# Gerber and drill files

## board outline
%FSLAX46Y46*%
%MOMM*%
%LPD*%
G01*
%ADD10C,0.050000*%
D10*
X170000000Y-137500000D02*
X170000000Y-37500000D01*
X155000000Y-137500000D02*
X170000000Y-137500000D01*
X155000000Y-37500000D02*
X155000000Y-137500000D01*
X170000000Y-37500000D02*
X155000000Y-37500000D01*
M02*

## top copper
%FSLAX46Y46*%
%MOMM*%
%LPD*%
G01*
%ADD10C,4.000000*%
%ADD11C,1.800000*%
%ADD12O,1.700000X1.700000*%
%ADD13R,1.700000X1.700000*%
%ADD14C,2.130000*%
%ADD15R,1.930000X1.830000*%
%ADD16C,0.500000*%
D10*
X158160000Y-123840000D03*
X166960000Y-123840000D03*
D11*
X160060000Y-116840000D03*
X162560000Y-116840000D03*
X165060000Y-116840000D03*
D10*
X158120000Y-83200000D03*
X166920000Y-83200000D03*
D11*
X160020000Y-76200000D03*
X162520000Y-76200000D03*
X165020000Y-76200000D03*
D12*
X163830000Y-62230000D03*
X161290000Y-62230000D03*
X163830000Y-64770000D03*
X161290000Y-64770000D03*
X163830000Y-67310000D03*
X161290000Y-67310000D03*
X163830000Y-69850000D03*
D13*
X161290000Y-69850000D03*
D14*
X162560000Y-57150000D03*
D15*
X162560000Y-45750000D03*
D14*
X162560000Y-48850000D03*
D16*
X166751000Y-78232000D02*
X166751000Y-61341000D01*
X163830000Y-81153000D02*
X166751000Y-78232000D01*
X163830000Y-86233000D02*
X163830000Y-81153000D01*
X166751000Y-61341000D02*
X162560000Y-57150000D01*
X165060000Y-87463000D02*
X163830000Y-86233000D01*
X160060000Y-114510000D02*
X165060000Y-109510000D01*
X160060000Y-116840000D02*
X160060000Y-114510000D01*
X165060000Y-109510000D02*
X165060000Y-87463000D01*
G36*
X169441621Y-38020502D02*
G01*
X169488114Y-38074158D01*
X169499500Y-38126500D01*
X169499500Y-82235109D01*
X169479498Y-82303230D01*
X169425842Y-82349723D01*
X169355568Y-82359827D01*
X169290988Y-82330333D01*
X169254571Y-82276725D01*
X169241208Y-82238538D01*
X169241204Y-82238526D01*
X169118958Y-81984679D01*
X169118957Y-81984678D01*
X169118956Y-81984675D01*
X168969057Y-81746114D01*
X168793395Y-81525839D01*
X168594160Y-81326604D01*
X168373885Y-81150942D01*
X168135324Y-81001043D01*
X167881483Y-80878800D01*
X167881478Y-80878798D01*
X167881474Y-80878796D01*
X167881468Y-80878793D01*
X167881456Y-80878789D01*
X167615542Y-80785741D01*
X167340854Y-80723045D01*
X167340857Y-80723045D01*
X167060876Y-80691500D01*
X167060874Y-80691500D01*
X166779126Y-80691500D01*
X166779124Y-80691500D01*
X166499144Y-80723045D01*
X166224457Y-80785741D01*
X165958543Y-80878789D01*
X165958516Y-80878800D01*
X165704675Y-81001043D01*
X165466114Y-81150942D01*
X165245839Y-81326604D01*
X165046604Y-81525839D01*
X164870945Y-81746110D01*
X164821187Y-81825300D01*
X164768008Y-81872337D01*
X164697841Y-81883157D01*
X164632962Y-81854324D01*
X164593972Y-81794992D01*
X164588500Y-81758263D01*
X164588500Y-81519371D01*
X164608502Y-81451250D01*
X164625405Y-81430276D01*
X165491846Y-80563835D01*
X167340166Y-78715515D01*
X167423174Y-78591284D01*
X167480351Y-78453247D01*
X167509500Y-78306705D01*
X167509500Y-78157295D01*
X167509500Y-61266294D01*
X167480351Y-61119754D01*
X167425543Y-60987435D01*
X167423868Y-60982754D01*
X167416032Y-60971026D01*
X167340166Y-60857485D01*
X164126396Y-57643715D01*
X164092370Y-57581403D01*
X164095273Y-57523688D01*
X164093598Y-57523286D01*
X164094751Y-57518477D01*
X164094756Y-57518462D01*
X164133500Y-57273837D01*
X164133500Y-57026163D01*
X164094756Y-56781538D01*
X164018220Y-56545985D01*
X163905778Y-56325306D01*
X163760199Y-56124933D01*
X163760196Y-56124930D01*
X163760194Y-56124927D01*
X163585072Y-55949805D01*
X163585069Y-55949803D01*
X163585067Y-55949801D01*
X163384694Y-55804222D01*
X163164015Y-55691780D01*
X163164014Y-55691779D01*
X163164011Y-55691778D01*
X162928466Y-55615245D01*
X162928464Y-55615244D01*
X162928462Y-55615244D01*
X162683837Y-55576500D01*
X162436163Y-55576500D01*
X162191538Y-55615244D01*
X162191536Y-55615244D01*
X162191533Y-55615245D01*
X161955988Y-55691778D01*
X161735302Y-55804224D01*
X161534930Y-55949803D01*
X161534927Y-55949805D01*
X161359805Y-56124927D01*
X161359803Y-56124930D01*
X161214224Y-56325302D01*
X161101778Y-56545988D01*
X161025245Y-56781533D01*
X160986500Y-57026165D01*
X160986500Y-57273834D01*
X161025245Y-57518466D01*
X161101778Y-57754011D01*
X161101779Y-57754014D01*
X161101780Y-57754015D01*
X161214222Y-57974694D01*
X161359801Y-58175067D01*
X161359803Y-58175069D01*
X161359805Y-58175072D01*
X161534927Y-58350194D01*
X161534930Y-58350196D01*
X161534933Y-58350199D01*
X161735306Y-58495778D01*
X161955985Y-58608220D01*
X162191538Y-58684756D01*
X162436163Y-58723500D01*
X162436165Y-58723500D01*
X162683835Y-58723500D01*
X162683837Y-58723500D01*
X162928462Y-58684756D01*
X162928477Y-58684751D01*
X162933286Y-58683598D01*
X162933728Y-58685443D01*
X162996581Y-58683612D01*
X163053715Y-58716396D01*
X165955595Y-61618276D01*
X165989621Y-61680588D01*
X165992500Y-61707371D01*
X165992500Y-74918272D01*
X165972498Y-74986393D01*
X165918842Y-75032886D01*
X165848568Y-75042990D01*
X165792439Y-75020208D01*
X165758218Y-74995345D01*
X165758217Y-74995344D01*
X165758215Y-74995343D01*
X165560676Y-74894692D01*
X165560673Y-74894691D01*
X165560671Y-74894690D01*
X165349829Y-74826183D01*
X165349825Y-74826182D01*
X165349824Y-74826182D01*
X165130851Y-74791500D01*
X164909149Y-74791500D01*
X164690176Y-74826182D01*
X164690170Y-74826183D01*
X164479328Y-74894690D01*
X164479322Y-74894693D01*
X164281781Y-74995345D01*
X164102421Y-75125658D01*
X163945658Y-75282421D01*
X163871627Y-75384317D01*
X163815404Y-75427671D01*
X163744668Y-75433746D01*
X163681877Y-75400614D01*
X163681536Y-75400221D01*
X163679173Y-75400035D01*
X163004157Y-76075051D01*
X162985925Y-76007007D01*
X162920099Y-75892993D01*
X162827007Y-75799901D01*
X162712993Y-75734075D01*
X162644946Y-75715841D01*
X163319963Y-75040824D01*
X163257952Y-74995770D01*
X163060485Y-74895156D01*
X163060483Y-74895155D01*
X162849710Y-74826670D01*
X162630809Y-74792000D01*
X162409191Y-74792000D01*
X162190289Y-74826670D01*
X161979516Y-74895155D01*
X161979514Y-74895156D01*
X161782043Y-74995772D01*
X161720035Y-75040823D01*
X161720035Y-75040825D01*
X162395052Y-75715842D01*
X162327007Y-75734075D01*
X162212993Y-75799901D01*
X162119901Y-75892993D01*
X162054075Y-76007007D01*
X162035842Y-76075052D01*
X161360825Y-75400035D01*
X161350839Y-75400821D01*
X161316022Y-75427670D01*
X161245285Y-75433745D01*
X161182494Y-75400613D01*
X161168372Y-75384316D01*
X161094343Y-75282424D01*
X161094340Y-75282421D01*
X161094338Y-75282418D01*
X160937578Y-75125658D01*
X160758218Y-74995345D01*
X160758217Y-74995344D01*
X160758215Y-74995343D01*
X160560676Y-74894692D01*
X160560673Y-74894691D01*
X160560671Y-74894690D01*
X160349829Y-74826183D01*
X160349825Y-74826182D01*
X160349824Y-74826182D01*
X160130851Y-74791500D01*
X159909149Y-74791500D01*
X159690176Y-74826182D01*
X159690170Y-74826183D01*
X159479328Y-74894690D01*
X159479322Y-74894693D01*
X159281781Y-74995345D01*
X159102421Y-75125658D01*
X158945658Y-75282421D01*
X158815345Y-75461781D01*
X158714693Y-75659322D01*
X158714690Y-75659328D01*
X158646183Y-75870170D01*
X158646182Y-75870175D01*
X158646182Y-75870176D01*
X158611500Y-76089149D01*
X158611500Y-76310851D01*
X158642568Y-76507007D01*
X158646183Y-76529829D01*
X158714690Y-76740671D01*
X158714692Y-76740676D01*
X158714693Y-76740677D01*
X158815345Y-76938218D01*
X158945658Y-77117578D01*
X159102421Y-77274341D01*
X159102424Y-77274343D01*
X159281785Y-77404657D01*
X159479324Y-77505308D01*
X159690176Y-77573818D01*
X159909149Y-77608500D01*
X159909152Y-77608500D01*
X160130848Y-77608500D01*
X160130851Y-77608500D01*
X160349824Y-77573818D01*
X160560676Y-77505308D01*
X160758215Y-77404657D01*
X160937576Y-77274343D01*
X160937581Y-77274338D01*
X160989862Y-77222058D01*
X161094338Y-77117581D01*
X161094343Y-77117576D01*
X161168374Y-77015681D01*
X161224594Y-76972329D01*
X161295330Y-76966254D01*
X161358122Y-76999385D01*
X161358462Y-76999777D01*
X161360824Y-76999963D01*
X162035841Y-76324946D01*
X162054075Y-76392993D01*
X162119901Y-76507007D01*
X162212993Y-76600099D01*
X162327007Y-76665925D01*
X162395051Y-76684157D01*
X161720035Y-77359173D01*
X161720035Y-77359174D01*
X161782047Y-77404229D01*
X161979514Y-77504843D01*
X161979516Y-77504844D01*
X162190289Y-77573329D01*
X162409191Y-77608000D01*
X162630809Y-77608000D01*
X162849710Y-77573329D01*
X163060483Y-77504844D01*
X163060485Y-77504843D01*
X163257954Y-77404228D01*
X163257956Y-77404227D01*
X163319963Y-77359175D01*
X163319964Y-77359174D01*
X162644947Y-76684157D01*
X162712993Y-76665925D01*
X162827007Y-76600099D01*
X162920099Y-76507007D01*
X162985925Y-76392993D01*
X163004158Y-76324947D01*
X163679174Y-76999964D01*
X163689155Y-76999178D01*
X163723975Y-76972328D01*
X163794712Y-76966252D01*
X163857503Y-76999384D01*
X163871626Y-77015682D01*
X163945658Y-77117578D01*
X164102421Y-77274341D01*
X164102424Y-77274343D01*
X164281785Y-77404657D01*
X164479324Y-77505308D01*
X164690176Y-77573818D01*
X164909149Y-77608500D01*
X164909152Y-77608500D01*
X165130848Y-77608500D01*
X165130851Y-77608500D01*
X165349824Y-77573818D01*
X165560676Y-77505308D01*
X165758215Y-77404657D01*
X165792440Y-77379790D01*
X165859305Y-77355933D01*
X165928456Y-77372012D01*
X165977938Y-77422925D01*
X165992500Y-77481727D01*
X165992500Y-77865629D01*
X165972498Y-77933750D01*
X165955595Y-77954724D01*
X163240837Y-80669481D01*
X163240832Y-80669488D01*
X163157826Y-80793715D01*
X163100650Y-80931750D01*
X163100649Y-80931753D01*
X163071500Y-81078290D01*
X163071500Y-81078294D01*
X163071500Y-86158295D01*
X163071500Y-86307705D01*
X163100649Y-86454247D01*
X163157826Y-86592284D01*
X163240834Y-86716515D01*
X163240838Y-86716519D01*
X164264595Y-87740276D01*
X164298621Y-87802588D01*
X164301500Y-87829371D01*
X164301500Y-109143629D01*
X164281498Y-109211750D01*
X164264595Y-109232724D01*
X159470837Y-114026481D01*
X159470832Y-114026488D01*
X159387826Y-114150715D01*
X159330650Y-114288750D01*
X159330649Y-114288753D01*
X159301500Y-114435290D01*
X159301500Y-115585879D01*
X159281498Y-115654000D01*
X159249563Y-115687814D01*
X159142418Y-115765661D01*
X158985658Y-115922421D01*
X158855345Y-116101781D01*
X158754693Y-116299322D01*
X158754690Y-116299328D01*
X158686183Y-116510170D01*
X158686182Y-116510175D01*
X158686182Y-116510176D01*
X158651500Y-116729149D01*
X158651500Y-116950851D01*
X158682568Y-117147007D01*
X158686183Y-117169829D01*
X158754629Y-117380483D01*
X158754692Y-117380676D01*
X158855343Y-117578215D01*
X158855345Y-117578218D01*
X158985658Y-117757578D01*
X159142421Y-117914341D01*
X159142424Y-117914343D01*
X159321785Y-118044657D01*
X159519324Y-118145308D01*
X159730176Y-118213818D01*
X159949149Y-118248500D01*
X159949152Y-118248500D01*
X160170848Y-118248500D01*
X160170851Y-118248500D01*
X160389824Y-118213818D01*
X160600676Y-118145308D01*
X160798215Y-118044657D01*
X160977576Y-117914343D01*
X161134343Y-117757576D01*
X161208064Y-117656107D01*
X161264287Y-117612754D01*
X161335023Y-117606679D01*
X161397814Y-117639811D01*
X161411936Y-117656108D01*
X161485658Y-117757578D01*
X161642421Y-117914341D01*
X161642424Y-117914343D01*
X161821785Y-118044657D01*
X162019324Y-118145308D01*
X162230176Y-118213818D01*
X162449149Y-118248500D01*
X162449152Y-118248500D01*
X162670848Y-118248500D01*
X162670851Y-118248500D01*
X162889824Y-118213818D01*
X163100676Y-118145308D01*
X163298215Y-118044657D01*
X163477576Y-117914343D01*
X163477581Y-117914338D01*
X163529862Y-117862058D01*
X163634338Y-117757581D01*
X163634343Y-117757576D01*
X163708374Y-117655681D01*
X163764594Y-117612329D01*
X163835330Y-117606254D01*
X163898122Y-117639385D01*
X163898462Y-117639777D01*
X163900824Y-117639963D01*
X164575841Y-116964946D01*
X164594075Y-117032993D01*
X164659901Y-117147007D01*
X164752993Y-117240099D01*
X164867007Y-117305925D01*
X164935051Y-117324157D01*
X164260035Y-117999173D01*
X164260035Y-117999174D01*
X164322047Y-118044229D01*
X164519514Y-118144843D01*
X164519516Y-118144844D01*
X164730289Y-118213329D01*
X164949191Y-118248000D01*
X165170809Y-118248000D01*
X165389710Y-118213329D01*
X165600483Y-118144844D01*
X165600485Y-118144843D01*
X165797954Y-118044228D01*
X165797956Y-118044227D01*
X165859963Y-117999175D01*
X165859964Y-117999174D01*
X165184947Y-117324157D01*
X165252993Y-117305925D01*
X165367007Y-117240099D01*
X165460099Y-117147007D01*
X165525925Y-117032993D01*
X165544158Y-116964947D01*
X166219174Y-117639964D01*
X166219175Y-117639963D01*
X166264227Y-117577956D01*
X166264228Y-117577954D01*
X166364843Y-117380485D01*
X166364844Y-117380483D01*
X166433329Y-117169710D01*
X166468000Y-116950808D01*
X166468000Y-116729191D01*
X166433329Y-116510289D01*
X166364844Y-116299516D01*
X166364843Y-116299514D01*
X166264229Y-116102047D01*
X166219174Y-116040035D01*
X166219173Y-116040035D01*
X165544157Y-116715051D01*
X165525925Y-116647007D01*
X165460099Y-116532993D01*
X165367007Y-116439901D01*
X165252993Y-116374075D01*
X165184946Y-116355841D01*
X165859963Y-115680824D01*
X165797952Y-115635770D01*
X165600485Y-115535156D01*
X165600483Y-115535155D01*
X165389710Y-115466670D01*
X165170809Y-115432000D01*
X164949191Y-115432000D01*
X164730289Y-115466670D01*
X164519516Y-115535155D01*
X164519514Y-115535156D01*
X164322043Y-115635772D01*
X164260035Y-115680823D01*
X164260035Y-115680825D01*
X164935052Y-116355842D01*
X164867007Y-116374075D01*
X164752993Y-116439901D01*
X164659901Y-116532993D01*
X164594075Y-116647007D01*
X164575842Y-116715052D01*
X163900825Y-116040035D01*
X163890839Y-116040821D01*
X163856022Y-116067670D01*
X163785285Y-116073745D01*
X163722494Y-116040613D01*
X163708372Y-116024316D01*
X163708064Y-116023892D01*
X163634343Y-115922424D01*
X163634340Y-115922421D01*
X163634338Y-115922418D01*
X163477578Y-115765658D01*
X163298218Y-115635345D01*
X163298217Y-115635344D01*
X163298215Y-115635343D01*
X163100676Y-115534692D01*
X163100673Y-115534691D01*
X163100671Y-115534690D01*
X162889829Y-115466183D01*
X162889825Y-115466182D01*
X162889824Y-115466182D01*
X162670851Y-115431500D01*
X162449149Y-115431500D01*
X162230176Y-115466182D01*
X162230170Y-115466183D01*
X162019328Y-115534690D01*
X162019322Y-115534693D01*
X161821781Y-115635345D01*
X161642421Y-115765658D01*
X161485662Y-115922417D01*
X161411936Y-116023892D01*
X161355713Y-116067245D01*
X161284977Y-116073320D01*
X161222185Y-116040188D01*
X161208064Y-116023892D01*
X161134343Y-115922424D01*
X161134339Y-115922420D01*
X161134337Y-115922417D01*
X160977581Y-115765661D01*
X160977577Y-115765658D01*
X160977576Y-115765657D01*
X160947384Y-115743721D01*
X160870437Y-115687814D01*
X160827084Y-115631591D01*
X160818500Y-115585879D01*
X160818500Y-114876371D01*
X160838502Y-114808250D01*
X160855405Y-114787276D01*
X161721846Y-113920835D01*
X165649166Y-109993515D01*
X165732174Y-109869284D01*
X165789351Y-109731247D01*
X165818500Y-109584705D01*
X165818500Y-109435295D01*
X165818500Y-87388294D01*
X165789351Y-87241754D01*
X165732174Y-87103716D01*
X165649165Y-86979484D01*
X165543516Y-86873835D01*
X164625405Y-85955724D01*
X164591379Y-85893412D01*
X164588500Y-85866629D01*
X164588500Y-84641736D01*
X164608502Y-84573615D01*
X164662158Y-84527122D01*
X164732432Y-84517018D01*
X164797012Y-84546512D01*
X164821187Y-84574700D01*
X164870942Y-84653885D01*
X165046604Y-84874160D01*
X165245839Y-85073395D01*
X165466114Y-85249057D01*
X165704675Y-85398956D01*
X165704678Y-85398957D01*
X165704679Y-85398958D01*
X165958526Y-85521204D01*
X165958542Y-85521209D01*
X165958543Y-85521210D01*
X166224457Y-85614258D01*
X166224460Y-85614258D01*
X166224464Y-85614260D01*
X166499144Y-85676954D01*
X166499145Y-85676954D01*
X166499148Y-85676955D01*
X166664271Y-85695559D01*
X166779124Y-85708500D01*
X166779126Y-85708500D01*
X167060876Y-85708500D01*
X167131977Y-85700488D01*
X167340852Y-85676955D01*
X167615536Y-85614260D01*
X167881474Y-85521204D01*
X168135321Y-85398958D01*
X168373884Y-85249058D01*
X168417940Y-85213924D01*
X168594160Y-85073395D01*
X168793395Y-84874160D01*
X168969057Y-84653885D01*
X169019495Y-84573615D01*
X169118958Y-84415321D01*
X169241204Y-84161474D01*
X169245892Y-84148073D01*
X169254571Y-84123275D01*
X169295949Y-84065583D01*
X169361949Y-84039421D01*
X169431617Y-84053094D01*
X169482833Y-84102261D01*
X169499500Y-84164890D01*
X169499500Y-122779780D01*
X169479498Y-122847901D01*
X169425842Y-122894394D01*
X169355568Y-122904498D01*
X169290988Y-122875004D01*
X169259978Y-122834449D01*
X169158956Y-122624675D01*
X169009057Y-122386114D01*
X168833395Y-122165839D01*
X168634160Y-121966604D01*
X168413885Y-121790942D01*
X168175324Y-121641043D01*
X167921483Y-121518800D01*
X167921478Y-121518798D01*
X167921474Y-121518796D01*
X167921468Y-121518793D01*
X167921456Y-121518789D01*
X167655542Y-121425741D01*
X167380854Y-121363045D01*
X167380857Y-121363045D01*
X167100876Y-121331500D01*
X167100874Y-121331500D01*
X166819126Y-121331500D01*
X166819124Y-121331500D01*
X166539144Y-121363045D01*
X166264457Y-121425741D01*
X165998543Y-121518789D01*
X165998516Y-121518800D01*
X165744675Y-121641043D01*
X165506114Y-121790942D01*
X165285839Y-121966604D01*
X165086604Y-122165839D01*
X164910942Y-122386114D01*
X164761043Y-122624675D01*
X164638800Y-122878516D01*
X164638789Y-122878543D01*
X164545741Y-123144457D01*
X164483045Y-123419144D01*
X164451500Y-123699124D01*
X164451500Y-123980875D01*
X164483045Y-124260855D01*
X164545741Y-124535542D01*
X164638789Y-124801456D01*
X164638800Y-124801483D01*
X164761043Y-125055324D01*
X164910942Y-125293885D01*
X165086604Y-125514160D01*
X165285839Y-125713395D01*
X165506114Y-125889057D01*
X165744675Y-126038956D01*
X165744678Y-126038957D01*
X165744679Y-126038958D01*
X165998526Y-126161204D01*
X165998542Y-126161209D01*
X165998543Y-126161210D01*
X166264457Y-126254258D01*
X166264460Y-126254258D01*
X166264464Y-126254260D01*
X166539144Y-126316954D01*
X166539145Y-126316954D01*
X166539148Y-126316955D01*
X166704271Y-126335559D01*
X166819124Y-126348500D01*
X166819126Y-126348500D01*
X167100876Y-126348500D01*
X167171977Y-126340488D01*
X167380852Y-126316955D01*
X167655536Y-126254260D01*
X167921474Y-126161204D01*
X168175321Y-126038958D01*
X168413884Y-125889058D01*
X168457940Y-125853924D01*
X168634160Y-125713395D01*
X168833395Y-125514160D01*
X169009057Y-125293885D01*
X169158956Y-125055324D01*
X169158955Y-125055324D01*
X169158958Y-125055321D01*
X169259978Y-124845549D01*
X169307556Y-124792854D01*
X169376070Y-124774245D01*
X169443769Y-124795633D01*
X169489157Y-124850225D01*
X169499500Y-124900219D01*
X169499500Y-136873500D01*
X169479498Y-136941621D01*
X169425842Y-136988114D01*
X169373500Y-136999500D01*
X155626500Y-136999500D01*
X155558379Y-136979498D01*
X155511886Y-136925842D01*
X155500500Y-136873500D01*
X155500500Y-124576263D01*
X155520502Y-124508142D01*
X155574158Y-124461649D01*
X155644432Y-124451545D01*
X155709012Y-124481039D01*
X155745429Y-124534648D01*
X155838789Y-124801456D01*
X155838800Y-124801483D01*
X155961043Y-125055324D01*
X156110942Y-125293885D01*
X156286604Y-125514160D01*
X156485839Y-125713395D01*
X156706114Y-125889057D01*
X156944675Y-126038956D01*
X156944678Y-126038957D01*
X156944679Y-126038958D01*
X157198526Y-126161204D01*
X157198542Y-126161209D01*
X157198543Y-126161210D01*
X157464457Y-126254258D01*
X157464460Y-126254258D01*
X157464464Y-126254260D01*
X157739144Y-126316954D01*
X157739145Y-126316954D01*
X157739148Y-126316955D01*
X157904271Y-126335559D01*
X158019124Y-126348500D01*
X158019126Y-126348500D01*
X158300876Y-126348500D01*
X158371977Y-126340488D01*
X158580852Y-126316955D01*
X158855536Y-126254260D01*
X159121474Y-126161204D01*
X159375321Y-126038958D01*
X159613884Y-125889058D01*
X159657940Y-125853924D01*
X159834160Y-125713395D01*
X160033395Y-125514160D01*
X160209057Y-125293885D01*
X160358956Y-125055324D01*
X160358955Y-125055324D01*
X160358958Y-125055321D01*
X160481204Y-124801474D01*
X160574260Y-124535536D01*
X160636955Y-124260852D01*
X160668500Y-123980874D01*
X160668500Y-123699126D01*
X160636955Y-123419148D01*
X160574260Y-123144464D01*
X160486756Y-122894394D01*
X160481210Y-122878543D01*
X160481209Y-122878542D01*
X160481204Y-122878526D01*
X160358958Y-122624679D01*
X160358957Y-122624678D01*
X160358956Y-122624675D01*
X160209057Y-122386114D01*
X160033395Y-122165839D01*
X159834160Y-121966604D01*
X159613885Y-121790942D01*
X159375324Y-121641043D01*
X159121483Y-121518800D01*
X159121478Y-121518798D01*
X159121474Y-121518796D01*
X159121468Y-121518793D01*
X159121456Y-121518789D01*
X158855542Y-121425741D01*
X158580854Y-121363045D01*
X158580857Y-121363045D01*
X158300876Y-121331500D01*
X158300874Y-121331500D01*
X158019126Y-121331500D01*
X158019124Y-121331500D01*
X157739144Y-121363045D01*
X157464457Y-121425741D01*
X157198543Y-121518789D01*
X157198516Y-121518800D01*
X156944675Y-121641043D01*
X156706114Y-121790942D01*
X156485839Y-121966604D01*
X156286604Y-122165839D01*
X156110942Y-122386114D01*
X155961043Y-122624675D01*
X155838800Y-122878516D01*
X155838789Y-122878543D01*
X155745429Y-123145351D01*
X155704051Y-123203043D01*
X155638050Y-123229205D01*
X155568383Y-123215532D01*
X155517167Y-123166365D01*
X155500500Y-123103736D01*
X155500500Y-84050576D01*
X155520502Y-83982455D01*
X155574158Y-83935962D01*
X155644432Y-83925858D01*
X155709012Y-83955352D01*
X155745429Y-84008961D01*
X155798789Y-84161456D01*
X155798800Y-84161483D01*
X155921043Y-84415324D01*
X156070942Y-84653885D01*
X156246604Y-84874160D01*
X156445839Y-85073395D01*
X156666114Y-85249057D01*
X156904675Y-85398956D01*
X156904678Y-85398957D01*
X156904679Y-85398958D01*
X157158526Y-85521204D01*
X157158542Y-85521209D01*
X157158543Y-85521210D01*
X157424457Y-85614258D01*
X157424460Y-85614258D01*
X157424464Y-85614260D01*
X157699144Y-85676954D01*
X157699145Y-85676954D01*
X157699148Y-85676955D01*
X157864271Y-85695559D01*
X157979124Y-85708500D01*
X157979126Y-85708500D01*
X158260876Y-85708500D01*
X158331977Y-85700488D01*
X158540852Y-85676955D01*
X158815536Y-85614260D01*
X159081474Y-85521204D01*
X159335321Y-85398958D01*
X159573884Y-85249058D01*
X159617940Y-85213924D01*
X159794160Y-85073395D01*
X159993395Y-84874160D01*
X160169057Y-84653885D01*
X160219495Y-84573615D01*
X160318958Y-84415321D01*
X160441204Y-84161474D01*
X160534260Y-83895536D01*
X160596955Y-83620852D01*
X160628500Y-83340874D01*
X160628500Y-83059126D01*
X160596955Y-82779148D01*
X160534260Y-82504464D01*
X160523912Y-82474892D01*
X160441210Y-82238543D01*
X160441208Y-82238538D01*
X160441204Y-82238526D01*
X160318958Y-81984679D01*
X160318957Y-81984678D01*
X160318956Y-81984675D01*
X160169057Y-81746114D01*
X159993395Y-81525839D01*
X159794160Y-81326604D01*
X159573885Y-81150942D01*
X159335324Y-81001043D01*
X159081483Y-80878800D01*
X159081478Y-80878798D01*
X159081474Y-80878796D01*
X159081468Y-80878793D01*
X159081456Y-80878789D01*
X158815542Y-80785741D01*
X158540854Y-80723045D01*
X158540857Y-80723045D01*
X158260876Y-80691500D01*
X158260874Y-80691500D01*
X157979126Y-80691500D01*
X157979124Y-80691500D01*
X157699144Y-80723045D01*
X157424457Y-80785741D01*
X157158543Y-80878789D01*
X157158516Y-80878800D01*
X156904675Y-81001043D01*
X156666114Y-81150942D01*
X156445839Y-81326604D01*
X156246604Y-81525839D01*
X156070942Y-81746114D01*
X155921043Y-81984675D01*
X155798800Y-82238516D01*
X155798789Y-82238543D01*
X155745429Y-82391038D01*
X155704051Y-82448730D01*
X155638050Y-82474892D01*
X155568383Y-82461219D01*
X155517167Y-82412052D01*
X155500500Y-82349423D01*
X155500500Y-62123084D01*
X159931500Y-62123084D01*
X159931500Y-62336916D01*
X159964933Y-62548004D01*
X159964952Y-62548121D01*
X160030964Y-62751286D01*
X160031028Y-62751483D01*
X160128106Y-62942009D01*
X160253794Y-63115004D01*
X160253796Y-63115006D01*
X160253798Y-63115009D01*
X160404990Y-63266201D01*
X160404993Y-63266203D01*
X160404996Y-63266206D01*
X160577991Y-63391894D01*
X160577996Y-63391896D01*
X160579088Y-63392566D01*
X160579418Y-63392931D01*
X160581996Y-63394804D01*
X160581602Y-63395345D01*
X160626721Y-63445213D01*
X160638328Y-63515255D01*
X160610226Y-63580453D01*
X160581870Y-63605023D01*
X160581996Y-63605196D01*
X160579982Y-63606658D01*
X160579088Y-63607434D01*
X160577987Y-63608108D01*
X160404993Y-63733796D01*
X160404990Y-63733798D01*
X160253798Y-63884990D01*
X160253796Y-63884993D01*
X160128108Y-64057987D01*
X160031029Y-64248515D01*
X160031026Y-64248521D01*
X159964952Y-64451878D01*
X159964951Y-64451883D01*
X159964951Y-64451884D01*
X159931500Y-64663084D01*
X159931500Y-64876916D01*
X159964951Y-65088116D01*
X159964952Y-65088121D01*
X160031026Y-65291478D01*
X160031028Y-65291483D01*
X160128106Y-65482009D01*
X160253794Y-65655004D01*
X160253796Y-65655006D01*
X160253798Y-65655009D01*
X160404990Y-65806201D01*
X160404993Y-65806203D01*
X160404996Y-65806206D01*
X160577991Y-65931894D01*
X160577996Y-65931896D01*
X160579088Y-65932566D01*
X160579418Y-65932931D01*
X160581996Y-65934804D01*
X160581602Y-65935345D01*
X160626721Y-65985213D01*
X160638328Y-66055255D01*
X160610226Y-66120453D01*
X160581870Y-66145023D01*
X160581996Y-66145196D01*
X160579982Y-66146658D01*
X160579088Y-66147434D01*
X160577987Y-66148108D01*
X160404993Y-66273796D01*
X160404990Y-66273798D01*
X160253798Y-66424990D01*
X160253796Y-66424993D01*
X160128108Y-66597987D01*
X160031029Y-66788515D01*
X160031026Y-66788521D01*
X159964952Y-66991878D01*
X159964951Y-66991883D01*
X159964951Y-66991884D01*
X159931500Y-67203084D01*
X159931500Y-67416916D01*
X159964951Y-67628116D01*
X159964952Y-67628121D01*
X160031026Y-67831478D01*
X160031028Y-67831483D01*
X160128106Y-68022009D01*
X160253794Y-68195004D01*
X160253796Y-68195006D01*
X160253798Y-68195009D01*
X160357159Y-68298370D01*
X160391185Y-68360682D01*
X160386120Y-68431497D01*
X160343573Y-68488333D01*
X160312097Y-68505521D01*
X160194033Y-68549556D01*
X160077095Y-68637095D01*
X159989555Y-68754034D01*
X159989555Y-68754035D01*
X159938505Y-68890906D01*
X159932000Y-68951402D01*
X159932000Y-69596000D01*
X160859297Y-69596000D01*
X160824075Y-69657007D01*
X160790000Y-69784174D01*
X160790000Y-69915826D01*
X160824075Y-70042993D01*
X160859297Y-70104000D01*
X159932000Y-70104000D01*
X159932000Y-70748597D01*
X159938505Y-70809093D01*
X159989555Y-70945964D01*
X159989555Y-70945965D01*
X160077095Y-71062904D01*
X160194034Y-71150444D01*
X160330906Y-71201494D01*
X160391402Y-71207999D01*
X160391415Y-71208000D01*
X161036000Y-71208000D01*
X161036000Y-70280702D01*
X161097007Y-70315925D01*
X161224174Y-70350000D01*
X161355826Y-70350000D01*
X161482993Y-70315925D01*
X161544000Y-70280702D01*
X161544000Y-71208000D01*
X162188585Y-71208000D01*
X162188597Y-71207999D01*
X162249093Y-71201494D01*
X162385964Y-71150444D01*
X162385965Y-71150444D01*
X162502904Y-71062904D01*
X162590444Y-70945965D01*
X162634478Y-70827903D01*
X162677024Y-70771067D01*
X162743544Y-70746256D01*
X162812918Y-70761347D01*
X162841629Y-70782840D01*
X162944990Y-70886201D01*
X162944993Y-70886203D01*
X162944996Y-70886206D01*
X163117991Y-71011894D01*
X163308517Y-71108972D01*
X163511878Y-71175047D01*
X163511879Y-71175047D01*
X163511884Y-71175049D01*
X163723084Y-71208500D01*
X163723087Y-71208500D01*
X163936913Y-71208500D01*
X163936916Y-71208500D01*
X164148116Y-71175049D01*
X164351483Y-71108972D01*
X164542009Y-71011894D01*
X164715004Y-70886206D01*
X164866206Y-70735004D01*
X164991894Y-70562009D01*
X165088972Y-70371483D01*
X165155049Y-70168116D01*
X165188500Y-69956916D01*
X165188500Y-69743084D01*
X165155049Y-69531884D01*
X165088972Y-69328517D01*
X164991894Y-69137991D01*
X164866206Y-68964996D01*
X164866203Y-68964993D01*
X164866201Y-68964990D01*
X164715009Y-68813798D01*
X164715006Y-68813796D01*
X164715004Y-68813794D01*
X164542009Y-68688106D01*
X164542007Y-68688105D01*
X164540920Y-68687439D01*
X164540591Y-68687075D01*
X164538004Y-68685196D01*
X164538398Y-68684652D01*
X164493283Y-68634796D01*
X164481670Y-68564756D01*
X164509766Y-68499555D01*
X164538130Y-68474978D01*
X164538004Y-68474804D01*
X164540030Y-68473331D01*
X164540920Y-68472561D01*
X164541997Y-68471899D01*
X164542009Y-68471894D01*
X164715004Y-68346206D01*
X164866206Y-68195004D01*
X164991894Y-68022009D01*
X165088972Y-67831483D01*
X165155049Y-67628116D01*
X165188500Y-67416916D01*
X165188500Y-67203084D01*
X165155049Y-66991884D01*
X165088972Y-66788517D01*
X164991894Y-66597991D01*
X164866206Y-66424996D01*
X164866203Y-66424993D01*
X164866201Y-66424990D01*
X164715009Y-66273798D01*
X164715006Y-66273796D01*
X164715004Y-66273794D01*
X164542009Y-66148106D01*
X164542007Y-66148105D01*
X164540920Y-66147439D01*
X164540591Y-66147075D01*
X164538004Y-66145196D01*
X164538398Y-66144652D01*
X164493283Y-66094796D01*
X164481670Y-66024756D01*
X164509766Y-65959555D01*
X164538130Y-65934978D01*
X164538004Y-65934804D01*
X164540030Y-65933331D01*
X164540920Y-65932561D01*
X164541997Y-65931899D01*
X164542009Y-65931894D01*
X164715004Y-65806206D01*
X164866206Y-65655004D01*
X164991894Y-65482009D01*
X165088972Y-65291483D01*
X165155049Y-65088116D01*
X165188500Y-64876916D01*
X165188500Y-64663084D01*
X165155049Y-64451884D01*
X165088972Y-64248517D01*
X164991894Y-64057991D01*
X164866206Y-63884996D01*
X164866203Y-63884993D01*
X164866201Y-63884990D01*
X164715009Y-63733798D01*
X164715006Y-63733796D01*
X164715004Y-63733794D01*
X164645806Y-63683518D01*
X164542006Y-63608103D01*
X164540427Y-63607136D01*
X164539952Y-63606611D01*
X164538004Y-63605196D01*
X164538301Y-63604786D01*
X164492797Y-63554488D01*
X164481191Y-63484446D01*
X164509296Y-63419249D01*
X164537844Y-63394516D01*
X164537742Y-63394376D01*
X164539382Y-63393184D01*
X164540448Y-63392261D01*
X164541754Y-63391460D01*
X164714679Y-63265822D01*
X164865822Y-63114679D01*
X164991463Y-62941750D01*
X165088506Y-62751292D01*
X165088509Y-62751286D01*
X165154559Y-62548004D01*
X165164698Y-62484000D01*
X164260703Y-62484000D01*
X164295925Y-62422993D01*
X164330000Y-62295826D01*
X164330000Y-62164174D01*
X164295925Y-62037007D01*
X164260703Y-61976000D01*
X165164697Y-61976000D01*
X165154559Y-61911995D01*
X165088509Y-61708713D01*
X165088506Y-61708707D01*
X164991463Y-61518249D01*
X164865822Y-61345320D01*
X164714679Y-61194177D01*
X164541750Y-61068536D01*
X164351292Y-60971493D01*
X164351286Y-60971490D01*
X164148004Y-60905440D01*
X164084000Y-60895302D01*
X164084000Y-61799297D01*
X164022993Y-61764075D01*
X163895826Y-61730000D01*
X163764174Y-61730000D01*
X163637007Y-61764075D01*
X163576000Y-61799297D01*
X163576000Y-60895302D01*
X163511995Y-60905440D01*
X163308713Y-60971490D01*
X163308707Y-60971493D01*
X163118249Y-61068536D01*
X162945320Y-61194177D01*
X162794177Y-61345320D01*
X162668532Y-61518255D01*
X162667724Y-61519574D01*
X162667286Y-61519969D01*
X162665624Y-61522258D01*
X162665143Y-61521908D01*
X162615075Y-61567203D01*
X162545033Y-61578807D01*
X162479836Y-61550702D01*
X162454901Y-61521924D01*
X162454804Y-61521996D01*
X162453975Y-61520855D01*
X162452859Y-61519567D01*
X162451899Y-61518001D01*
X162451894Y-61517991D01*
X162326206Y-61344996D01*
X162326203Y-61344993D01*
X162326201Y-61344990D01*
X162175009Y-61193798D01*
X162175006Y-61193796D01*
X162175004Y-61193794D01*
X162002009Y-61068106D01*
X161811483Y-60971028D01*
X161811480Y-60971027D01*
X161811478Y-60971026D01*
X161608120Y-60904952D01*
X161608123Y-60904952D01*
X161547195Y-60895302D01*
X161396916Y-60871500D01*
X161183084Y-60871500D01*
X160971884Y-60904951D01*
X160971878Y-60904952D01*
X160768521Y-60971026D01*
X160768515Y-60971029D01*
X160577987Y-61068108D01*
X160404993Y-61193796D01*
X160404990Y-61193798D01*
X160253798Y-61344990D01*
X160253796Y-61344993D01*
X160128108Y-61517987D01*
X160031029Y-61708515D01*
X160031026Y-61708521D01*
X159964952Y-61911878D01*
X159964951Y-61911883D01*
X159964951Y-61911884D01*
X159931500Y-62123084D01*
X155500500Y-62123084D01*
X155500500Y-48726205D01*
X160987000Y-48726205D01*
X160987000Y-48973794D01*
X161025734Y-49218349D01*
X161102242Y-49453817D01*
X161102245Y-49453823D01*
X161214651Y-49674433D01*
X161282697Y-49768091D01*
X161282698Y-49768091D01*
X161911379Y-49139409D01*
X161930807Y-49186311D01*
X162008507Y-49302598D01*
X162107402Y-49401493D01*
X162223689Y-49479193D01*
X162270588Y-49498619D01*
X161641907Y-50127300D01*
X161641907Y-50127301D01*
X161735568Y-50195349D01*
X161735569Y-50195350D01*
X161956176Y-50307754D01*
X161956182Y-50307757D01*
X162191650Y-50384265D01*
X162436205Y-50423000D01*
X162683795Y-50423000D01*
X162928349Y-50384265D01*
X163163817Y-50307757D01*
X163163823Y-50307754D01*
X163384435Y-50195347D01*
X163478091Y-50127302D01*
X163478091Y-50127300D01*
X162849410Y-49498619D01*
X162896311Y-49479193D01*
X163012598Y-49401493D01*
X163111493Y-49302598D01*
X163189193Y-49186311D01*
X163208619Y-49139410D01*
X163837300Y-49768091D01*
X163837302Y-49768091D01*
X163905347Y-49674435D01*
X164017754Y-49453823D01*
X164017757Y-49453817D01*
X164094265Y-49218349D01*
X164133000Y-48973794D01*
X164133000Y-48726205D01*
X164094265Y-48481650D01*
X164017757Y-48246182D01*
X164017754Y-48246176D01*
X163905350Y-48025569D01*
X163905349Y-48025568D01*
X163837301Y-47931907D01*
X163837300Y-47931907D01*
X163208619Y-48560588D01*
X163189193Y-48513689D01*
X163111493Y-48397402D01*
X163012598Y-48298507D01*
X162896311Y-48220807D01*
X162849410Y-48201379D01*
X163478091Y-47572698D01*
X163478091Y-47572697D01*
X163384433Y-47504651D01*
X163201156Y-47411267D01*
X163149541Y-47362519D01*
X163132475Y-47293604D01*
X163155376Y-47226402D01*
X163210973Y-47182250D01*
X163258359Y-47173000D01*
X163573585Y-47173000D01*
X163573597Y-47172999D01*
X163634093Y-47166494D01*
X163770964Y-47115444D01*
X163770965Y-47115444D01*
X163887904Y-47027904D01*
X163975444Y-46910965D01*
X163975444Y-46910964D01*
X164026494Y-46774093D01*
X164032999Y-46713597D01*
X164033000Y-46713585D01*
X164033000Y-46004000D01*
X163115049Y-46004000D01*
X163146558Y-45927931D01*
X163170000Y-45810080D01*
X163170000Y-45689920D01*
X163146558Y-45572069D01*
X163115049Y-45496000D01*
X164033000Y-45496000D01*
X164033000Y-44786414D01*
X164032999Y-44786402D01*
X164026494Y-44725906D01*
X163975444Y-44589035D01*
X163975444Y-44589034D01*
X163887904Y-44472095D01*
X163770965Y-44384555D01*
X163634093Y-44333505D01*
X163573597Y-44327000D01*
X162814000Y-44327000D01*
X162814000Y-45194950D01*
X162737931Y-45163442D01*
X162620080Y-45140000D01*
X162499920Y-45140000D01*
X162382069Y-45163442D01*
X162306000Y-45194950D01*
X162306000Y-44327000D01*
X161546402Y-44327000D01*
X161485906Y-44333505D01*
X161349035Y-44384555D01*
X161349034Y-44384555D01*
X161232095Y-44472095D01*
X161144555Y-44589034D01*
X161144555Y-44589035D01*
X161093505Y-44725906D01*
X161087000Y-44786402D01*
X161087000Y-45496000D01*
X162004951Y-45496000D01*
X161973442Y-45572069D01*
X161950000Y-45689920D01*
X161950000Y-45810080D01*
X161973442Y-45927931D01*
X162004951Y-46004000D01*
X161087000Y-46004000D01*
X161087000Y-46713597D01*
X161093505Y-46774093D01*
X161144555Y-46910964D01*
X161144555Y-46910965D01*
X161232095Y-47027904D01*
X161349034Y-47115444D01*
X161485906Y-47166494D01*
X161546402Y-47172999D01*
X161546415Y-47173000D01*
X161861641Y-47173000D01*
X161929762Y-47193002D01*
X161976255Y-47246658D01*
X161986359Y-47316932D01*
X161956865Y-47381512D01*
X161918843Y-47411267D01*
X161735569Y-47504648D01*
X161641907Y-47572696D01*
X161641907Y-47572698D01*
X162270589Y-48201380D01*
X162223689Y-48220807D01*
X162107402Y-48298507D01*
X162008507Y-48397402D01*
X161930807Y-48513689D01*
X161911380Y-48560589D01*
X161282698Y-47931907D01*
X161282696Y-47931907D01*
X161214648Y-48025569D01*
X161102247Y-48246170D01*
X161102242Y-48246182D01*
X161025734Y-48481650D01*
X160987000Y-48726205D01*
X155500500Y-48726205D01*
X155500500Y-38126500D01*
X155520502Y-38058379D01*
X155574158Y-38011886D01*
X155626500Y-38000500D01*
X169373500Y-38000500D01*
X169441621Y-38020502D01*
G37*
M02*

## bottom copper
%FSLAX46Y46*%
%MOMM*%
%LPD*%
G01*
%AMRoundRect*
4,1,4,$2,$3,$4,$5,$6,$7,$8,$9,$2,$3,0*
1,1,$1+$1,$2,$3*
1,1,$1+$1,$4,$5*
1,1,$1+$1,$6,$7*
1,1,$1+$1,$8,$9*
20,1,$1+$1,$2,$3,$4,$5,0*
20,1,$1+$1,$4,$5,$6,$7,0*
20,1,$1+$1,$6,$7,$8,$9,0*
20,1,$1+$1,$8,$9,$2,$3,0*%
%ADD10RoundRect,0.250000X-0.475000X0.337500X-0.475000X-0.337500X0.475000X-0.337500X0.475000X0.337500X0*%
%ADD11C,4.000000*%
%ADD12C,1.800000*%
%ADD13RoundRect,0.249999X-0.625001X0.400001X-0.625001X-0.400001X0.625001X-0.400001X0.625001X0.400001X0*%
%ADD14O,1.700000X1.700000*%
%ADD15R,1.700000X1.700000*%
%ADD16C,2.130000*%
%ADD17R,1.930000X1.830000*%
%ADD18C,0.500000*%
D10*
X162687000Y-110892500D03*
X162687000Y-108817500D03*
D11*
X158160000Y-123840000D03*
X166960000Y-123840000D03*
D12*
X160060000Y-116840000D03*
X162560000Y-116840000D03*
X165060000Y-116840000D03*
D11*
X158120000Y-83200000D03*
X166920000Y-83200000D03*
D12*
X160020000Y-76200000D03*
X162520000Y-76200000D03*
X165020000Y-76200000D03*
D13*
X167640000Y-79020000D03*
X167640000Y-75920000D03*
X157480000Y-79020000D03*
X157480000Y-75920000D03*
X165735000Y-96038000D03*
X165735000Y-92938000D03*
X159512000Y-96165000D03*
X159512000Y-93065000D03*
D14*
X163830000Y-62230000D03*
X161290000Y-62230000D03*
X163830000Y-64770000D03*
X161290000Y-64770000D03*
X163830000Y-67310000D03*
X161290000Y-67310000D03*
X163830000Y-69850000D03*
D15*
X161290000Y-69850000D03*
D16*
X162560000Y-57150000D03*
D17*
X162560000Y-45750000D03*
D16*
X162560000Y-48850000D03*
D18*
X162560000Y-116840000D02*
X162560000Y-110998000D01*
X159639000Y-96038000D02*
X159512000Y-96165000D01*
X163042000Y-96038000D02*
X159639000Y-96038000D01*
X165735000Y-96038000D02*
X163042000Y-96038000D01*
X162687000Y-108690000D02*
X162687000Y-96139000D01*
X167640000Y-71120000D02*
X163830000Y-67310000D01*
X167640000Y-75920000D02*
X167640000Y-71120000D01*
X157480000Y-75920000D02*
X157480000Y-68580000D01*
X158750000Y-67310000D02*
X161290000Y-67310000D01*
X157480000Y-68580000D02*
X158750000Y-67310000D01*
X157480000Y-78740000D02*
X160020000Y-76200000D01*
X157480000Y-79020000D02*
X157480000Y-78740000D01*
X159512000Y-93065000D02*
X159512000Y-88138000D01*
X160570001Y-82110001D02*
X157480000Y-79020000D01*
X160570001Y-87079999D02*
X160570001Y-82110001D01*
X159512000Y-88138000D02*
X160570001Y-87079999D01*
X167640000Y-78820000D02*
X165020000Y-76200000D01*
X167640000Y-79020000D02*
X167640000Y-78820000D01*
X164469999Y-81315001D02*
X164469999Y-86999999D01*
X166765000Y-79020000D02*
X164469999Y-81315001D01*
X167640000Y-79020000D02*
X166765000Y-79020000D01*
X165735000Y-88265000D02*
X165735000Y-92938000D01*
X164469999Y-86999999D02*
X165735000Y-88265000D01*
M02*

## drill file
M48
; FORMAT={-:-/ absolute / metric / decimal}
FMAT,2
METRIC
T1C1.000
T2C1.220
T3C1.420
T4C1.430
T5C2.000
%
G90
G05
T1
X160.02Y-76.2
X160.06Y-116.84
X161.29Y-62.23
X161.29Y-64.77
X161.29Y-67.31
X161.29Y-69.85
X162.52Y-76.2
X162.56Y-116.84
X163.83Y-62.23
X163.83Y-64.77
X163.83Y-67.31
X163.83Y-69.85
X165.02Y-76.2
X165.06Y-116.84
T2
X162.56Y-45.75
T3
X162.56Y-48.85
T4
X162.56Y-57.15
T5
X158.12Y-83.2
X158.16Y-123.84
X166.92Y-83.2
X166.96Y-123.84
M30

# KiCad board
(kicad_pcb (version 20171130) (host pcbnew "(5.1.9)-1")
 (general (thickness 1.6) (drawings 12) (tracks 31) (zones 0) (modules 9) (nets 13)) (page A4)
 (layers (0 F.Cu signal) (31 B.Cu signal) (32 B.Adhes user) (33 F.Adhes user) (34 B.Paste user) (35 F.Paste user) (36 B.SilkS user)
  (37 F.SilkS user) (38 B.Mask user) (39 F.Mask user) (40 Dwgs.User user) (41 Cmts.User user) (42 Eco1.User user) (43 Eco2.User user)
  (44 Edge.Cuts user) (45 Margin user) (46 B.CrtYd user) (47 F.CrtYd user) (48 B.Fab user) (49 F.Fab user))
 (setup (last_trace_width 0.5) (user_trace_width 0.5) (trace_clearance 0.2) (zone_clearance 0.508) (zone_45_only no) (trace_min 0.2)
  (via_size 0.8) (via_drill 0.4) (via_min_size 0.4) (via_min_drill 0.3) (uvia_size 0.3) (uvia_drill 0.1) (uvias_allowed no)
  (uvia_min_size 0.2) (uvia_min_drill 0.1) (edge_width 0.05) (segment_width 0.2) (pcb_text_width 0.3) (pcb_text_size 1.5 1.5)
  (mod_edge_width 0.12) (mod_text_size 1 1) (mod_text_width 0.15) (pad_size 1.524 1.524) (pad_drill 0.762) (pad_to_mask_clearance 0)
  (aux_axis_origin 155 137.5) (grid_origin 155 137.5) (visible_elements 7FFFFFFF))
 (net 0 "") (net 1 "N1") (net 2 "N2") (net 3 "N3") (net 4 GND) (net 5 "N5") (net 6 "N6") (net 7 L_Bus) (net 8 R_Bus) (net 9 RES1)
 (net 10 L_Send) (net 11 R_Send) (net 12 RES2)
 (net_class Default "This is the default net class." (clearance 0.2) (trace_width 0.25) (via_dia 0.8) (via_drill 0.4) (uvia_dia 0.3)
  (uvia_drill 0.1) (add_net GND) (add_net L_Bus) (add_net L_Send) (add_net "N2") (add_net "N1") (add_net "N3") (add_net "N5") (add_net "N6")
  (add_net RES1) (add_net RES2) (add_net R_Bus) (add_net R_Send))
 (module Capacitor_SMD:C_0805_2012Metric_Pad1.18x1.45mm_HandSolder (layer B.Cu) (at 162.687 109.855 270)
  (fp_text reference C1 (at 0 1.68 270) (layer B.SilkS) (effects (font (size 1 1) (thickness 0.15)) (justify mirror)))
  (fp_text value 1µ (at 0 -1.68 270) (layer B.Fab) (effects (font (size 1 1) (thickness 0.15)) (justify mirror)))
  (pad 2 smd roundrect (at 1.0375 0 270) (size 1.175 1.45) (layers B.Cu B.Paste B.Mask) (roundrect_rratio 0.2127659574468085) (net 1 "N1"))
  (pad 1 smd roundrect (at -1.0375 0 270) (size 1.175 1.45) (layers B.Cu B.Paste B.Mask) (roundrect_rratio 0.2127659574468085) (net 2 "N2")))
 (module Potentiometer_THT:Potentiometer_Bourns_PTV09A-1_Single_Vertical (layer F.Cu) (at 160.06 116.84 270)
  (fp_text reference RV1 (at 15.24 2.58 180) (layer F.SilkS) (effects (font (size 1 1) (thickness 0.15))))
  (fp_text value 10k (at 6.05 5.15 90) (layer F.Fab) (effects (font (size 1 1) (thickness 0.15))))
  (pad "" np_thru_hole circle (at 7 1.9 270) (size 4 4) (drill 2) (layers *.Cu *.Mask))
  (pad "" np_thru_hole circle (at 7 -6.9 270) (size 4 4) (drill 2) (layers *.Cu *.Mask))
  (pad 1 thru_hole circle (at 0 0 270) (size 1.8 1.8) (drill 1) (layers *.Cu *.Mask) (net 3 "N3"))
  (pad 2 thru_hole circle (at 0 -2.5 270) (size 1.8 1.8) (drill 1) (layers *.Cu *.Mask) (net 1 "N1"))
  (pad 3 thru_hole circle (at 0 -5 270) (size 1.8 1.8) (drill 1) (layers *.Cu *.Mask) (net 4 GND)))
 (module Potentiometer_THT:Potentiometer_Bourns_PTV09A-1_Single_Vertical (layer F.Cu) (at 160.02 76.2 270)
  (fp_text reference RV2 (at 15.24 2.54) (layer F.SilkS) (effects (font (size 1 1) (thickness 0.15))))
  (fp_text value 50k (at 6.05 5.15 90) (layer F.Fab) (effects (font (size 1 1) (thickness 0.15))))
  (pad "" np_thru_hole circle (at 7 1.9 270) (size 4 4) (drill 2) (layers *.Cu *.Mask))
  (pad "" np_thru_hole circle (at 7 -6.9 270) (size 4 4) (drill 2) (layers *.Cu *.Mask))
  (pad 1 thru_hole circle (at 0 0 270) (size 1.8 1.8) (drill 1) (layers *.Cu *.Mask) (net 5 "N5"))
  (pad 2 thru_hole circle (at 0 -2.5 270) (size 1.8 1.8) (drill 1) (layers *.Cu *.Mask) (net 4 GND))
  (pad 3 thru_hole circle (at 0 -5 270) (size 1.8 1.8) (drill 1) (layers *.Cu *.Mask) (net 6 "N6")))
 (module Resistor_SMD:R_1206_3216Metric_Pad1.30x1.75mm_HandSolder (layer B.Cu) (at 167.64 77.47 270)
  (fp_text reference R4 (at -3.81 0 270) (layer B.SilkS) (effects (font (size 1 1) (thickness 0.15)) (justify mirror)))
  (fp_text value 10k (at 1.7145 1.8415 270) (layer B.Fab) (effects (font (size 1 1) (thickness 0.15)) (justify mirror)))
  (pad 2 smd roundrect (at 1.55 0 270) (size 1.3 1.75) (layers B.Cu B.Paste B.Mask) (roundrect_rratio 0.1923069230769231) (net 6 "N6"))
  (pad 1 smd roundrect (at -1.55 0 270) (size 1.3 1.75) (layers B.Cu B.Paste B.Mask) (roundrect_rratio 0.1923069230769231) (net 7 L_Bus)))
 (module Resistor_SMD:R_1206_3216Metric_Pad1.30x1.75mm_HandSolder (layer B.Cu) (at 157.48 77.47 270)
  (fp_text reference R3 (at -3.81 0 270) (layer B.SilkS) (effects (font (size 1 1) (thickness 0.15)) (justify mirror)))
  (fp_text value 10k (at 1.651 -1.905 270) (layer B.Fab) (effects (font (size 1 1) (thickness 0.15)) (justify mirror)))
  (pad 2 smd roundrect (at 1.55 0 270) (size 1.3 1.75) (layers B.Cu B.Paste B.Mask) (roundrect_rratio 0.1923069230769231) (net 5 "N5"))
  (pad 1 smd roundrect (at -1.55 0 270) (size 1.3 1.75) (layers B.Cu B.Paste B.Mask) (roundrect_rratio 0.1923069230769231) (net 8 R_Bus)))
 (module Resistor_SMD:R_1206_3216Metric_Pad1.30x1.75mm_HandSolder (layer B.Cu) (at 165.735 94.488 270)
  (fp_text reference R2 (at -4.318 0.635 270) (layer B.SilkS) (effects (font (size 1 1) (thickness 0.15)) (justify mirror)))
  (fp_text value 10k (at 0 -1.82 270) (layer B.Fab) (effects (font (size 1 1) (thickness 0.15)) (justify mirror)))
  (pad 2 smd roundrect (at 1.55 0 270) (size 1.3 1.75) (layers B.Cu B.Paste B.Mask) (roundrect_rratio 0.1923069230769231) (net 2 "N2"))
  (pad 1 smd roundrect (at -1.55 0 270) (size 1.3 1.75) (layers B.Cu B.Paste B.Mask) (roundrect_rratio 0.1923069230769231) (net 6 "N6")))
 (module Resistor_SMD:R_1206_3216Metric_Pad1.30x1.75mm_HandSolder (layer B.Cu) (at 159.512 94.615 270)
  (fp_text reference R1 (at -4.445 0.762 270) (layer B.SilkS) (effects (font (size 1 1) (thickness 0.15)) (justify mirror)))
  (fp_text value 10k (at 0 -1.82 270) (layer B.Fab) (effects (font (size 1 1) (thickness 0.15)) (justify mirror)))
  (pad 2 smd roundrect (at 1.55 0 270) (size 1.3 1.75) (layers B.Cu B.Paste B.Mask) (roundrect_rratio 0.1923069230769231) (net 2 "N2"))
  (pad 1 smd roundrect (at -1.55 0 270) (size 1.3 1.75) (layers B.Cu B.Paste B.Mask) (roundrect_rratio 0.1923069230769231) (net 5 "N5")))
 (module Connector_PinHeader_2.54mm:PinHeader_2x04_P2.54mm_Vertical (layer B.Cu) (at 161.29 69.85)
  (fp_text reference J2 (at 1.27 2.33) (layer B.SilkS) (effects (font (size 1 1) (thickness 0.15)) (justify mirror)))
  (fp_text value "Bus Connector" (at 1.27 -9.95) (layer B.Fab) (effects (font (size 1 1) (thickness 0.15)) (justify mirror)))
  (pad 8 thru_hole oval (at 2.54 -7.62) (size 1.7 1.7) (drill 1) (layers *.Cu *.Mask) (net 4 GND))
  (pad 7 thru_hole oval (at 0 -7.62) (size 1.7 1.7) (drill 1) (layers *.Cu *.Mask) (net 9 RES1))
  (pad 6 thru_hole oval (at 2.54 -5.08) (size 1.7 1.7) (drill 1) (layers *.Cu *.Mask) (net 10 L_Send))
  (pad 5 thru_hole oval (at 0 -5.08) (size 1.7 1.7) (drill 1) (layers *.Cu *.Mask) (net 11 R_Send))
  (pad 4 thru_hole oval (at 2.54 -2.54) (size 1.7 1.7) (drill 1) (layers *.Cu *.Mask) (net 7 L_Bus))
  (pad 3 thru_hole oval (at 0 -2.54) (size 1.7 1.7) (drill 1) (layers *.Cu *.Mask) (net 8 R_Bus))
  (pad 2 thru_hole oval (at 2.54 0) (size 1.7 1.7) (drill 1) (layers *.Cu *.Mask) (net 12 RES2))
  (pad 1 thru_hole rect (at 0 0) (size 1.7 1.7) (drill 1) (layers *.Cu *.Mask) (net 4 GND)))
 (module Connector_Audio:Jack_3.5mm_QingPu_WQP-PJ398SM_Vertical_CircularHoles (layer F.Cu) (at 162.56 45.75)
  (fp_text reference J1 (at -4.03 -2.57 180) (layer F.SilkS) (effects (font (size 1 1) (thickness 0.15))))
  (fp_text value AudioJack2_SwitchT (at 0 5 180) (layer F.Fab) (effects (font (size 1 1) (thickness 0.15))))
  (pad T thru_hole circle (at 0 11.4 180) (size 2.13 2.13) (drill 1.43) (layers *.Cu *.Mask) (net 3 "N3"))
  (pad S thru_hole rect (at 0 0 180) (size 1.93 1.83) (drill 1.22) (layers *.Cu *.Mask) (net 4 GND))
  (pad TN thru_hole circle (at 0 3.1 180) (size 2.13 2.13) (drill 1.42) (layers *.Cu *.Mask) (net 4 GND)))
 (gr_line (start 170 137.5) (end 170 37.5) (layer Edge.Cuts) (width 0.05))
 (gr_line (start 155 137.5) (end 170 137.5) (layer Edge.Cuts) (width 0.05))
 (gr_line (start 155 37.5) (end 155 137.5) (layer Edge.Cuts) (width 0.05))
 (gr_line (start 170 37.5) (end 155 37.5) (layer Edge.Cuts) (width 0.05))
 (segment (start 162.56 116.84) (end 162.56 110.998) (width 0.5) (layer B.Cu) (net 1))
 (segment (start 159.639 96.038) (end 159.512 96.165) (width 0.5) (layer B.Cu) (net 2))
 (segment (start 163.042 96.038) (end 159.639 96.038) (width 0.5) (layer B.Cu) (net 2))
 (segment (start 165.735 96.038) (end 163.042 96.038) (width 0.5) (layer B.Cu) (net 2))
 (segment (start 162.687 108.69) (end 162.687 96.139) (width 0.5) (layer B.Cu) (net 2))
 (segment (start 166.751 78.232) (end 166.751 61.341) (width 0.5) (layer F.Cu) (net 3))
 (segment (start 163.83 81.153) (end 166.751 78.232) (width 0.5) (layer F.Cu) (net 3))
 (segment (start 163.83 86.233) (end 163.83 81.153) (width 0.5) (layer F.Cu) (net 3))
 (segment (start 166.751 61.341) (end 162.56 57.15) (width 0.5) (layer F.Cu) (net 3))
 (segment (start 165.06 87.463) (end 163.83 86.233) (width 0.5) (layer F.Cu) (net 3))
 (segment (start 160.06 114.51) (end 165.06 109.51) (width 0.5) (layer F.Cu) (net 3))
 (segment (start 160.06 116.84) (end 160.06 114.51) (width 0.5) (layer F.Cu) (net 3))
 (segment (start 165.06 109.51) (end 165.06 87.463) (width 0.5) (layer F.Cu) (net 3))
 (segment (start 167.64 71.12) (end 163.83 67.31) (width 0.5) (layer B.Cu) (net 7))
 (segment (start 167.64 75.92) (end 167.64 71.12) (width 0.5) (layer B.Cu) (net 7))
 (segment (start 157.48 75.92) (end 157.48 68.58) (width 0.5) (layer B.Cu) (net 8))
 (segment (start 158.75 67.31) (end 161.29 67.31) (width 0.5) (layer B.Cu) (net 8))
 (segment (start 157.48 68.58) (end 158.75 67.31) (width 0.5) (layer B.Cu) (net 8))
 (segment (start 157.48 78.74) (end 160.02 76.2) (width 0.5) (layer B.Cu) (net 5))
 (segment (start 157.48 79.02) (end 157.48 78.74) (width 0.5) (layer B.Cu) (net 5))
 (segment (start 159.512 93.065) (end 159.512 88.138) (width 0.5) (layer B.Cu) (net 5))
 (segment (start 160.570001 82.110001) (end 157.48 79.02) (width 0.5) (layer B.Cu) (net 5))
 (segment (start 160.570001 87.079999) (end 160.570001 82.110001) (width 0.5) (layer B.Cu) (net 5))
 (segment (start 159.512 88.138) (end 160.570001 87.079999) (width 0.5) (layer B.Cu) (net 5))
 (segment (start 167.64 78.82) (end 165.02 76.2) (width 0.5) (layer B.Cu) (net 6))
 (segment (start 167.64 79.02) (end 167.64 78.82) (width 0.5) (layer B.Cu) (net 6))
 (segment (start 164.469999 81.315001) (end 164.469999 86.999999) (width 0.5) (layer B.Cu) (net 6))
 (segment (start 166.765 79.02) (end 164.469999 81.315001) (width 0.5) (layer B.Cu) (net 6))
 (segment (start 167.64 79.02) (end 166.765 79.02) (width 0.5) (layer B.Cu) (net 6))
 (segment (start 165.735 88.265) (end 165.735 92.938) (width 0.5) (layer B.Cu) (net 6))
 (segment (start 164.469999 86.999999) (end 165.735 88.265) (width 0.5) (layer B.Cu) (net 6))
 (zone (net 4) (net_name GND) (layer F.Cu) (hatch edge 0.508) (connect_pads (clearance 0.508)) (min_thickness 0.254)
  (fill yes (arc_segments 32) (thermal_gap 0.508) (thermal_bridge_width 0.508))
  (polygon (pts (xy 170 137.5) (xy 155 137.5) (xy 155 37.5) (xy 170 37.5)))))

